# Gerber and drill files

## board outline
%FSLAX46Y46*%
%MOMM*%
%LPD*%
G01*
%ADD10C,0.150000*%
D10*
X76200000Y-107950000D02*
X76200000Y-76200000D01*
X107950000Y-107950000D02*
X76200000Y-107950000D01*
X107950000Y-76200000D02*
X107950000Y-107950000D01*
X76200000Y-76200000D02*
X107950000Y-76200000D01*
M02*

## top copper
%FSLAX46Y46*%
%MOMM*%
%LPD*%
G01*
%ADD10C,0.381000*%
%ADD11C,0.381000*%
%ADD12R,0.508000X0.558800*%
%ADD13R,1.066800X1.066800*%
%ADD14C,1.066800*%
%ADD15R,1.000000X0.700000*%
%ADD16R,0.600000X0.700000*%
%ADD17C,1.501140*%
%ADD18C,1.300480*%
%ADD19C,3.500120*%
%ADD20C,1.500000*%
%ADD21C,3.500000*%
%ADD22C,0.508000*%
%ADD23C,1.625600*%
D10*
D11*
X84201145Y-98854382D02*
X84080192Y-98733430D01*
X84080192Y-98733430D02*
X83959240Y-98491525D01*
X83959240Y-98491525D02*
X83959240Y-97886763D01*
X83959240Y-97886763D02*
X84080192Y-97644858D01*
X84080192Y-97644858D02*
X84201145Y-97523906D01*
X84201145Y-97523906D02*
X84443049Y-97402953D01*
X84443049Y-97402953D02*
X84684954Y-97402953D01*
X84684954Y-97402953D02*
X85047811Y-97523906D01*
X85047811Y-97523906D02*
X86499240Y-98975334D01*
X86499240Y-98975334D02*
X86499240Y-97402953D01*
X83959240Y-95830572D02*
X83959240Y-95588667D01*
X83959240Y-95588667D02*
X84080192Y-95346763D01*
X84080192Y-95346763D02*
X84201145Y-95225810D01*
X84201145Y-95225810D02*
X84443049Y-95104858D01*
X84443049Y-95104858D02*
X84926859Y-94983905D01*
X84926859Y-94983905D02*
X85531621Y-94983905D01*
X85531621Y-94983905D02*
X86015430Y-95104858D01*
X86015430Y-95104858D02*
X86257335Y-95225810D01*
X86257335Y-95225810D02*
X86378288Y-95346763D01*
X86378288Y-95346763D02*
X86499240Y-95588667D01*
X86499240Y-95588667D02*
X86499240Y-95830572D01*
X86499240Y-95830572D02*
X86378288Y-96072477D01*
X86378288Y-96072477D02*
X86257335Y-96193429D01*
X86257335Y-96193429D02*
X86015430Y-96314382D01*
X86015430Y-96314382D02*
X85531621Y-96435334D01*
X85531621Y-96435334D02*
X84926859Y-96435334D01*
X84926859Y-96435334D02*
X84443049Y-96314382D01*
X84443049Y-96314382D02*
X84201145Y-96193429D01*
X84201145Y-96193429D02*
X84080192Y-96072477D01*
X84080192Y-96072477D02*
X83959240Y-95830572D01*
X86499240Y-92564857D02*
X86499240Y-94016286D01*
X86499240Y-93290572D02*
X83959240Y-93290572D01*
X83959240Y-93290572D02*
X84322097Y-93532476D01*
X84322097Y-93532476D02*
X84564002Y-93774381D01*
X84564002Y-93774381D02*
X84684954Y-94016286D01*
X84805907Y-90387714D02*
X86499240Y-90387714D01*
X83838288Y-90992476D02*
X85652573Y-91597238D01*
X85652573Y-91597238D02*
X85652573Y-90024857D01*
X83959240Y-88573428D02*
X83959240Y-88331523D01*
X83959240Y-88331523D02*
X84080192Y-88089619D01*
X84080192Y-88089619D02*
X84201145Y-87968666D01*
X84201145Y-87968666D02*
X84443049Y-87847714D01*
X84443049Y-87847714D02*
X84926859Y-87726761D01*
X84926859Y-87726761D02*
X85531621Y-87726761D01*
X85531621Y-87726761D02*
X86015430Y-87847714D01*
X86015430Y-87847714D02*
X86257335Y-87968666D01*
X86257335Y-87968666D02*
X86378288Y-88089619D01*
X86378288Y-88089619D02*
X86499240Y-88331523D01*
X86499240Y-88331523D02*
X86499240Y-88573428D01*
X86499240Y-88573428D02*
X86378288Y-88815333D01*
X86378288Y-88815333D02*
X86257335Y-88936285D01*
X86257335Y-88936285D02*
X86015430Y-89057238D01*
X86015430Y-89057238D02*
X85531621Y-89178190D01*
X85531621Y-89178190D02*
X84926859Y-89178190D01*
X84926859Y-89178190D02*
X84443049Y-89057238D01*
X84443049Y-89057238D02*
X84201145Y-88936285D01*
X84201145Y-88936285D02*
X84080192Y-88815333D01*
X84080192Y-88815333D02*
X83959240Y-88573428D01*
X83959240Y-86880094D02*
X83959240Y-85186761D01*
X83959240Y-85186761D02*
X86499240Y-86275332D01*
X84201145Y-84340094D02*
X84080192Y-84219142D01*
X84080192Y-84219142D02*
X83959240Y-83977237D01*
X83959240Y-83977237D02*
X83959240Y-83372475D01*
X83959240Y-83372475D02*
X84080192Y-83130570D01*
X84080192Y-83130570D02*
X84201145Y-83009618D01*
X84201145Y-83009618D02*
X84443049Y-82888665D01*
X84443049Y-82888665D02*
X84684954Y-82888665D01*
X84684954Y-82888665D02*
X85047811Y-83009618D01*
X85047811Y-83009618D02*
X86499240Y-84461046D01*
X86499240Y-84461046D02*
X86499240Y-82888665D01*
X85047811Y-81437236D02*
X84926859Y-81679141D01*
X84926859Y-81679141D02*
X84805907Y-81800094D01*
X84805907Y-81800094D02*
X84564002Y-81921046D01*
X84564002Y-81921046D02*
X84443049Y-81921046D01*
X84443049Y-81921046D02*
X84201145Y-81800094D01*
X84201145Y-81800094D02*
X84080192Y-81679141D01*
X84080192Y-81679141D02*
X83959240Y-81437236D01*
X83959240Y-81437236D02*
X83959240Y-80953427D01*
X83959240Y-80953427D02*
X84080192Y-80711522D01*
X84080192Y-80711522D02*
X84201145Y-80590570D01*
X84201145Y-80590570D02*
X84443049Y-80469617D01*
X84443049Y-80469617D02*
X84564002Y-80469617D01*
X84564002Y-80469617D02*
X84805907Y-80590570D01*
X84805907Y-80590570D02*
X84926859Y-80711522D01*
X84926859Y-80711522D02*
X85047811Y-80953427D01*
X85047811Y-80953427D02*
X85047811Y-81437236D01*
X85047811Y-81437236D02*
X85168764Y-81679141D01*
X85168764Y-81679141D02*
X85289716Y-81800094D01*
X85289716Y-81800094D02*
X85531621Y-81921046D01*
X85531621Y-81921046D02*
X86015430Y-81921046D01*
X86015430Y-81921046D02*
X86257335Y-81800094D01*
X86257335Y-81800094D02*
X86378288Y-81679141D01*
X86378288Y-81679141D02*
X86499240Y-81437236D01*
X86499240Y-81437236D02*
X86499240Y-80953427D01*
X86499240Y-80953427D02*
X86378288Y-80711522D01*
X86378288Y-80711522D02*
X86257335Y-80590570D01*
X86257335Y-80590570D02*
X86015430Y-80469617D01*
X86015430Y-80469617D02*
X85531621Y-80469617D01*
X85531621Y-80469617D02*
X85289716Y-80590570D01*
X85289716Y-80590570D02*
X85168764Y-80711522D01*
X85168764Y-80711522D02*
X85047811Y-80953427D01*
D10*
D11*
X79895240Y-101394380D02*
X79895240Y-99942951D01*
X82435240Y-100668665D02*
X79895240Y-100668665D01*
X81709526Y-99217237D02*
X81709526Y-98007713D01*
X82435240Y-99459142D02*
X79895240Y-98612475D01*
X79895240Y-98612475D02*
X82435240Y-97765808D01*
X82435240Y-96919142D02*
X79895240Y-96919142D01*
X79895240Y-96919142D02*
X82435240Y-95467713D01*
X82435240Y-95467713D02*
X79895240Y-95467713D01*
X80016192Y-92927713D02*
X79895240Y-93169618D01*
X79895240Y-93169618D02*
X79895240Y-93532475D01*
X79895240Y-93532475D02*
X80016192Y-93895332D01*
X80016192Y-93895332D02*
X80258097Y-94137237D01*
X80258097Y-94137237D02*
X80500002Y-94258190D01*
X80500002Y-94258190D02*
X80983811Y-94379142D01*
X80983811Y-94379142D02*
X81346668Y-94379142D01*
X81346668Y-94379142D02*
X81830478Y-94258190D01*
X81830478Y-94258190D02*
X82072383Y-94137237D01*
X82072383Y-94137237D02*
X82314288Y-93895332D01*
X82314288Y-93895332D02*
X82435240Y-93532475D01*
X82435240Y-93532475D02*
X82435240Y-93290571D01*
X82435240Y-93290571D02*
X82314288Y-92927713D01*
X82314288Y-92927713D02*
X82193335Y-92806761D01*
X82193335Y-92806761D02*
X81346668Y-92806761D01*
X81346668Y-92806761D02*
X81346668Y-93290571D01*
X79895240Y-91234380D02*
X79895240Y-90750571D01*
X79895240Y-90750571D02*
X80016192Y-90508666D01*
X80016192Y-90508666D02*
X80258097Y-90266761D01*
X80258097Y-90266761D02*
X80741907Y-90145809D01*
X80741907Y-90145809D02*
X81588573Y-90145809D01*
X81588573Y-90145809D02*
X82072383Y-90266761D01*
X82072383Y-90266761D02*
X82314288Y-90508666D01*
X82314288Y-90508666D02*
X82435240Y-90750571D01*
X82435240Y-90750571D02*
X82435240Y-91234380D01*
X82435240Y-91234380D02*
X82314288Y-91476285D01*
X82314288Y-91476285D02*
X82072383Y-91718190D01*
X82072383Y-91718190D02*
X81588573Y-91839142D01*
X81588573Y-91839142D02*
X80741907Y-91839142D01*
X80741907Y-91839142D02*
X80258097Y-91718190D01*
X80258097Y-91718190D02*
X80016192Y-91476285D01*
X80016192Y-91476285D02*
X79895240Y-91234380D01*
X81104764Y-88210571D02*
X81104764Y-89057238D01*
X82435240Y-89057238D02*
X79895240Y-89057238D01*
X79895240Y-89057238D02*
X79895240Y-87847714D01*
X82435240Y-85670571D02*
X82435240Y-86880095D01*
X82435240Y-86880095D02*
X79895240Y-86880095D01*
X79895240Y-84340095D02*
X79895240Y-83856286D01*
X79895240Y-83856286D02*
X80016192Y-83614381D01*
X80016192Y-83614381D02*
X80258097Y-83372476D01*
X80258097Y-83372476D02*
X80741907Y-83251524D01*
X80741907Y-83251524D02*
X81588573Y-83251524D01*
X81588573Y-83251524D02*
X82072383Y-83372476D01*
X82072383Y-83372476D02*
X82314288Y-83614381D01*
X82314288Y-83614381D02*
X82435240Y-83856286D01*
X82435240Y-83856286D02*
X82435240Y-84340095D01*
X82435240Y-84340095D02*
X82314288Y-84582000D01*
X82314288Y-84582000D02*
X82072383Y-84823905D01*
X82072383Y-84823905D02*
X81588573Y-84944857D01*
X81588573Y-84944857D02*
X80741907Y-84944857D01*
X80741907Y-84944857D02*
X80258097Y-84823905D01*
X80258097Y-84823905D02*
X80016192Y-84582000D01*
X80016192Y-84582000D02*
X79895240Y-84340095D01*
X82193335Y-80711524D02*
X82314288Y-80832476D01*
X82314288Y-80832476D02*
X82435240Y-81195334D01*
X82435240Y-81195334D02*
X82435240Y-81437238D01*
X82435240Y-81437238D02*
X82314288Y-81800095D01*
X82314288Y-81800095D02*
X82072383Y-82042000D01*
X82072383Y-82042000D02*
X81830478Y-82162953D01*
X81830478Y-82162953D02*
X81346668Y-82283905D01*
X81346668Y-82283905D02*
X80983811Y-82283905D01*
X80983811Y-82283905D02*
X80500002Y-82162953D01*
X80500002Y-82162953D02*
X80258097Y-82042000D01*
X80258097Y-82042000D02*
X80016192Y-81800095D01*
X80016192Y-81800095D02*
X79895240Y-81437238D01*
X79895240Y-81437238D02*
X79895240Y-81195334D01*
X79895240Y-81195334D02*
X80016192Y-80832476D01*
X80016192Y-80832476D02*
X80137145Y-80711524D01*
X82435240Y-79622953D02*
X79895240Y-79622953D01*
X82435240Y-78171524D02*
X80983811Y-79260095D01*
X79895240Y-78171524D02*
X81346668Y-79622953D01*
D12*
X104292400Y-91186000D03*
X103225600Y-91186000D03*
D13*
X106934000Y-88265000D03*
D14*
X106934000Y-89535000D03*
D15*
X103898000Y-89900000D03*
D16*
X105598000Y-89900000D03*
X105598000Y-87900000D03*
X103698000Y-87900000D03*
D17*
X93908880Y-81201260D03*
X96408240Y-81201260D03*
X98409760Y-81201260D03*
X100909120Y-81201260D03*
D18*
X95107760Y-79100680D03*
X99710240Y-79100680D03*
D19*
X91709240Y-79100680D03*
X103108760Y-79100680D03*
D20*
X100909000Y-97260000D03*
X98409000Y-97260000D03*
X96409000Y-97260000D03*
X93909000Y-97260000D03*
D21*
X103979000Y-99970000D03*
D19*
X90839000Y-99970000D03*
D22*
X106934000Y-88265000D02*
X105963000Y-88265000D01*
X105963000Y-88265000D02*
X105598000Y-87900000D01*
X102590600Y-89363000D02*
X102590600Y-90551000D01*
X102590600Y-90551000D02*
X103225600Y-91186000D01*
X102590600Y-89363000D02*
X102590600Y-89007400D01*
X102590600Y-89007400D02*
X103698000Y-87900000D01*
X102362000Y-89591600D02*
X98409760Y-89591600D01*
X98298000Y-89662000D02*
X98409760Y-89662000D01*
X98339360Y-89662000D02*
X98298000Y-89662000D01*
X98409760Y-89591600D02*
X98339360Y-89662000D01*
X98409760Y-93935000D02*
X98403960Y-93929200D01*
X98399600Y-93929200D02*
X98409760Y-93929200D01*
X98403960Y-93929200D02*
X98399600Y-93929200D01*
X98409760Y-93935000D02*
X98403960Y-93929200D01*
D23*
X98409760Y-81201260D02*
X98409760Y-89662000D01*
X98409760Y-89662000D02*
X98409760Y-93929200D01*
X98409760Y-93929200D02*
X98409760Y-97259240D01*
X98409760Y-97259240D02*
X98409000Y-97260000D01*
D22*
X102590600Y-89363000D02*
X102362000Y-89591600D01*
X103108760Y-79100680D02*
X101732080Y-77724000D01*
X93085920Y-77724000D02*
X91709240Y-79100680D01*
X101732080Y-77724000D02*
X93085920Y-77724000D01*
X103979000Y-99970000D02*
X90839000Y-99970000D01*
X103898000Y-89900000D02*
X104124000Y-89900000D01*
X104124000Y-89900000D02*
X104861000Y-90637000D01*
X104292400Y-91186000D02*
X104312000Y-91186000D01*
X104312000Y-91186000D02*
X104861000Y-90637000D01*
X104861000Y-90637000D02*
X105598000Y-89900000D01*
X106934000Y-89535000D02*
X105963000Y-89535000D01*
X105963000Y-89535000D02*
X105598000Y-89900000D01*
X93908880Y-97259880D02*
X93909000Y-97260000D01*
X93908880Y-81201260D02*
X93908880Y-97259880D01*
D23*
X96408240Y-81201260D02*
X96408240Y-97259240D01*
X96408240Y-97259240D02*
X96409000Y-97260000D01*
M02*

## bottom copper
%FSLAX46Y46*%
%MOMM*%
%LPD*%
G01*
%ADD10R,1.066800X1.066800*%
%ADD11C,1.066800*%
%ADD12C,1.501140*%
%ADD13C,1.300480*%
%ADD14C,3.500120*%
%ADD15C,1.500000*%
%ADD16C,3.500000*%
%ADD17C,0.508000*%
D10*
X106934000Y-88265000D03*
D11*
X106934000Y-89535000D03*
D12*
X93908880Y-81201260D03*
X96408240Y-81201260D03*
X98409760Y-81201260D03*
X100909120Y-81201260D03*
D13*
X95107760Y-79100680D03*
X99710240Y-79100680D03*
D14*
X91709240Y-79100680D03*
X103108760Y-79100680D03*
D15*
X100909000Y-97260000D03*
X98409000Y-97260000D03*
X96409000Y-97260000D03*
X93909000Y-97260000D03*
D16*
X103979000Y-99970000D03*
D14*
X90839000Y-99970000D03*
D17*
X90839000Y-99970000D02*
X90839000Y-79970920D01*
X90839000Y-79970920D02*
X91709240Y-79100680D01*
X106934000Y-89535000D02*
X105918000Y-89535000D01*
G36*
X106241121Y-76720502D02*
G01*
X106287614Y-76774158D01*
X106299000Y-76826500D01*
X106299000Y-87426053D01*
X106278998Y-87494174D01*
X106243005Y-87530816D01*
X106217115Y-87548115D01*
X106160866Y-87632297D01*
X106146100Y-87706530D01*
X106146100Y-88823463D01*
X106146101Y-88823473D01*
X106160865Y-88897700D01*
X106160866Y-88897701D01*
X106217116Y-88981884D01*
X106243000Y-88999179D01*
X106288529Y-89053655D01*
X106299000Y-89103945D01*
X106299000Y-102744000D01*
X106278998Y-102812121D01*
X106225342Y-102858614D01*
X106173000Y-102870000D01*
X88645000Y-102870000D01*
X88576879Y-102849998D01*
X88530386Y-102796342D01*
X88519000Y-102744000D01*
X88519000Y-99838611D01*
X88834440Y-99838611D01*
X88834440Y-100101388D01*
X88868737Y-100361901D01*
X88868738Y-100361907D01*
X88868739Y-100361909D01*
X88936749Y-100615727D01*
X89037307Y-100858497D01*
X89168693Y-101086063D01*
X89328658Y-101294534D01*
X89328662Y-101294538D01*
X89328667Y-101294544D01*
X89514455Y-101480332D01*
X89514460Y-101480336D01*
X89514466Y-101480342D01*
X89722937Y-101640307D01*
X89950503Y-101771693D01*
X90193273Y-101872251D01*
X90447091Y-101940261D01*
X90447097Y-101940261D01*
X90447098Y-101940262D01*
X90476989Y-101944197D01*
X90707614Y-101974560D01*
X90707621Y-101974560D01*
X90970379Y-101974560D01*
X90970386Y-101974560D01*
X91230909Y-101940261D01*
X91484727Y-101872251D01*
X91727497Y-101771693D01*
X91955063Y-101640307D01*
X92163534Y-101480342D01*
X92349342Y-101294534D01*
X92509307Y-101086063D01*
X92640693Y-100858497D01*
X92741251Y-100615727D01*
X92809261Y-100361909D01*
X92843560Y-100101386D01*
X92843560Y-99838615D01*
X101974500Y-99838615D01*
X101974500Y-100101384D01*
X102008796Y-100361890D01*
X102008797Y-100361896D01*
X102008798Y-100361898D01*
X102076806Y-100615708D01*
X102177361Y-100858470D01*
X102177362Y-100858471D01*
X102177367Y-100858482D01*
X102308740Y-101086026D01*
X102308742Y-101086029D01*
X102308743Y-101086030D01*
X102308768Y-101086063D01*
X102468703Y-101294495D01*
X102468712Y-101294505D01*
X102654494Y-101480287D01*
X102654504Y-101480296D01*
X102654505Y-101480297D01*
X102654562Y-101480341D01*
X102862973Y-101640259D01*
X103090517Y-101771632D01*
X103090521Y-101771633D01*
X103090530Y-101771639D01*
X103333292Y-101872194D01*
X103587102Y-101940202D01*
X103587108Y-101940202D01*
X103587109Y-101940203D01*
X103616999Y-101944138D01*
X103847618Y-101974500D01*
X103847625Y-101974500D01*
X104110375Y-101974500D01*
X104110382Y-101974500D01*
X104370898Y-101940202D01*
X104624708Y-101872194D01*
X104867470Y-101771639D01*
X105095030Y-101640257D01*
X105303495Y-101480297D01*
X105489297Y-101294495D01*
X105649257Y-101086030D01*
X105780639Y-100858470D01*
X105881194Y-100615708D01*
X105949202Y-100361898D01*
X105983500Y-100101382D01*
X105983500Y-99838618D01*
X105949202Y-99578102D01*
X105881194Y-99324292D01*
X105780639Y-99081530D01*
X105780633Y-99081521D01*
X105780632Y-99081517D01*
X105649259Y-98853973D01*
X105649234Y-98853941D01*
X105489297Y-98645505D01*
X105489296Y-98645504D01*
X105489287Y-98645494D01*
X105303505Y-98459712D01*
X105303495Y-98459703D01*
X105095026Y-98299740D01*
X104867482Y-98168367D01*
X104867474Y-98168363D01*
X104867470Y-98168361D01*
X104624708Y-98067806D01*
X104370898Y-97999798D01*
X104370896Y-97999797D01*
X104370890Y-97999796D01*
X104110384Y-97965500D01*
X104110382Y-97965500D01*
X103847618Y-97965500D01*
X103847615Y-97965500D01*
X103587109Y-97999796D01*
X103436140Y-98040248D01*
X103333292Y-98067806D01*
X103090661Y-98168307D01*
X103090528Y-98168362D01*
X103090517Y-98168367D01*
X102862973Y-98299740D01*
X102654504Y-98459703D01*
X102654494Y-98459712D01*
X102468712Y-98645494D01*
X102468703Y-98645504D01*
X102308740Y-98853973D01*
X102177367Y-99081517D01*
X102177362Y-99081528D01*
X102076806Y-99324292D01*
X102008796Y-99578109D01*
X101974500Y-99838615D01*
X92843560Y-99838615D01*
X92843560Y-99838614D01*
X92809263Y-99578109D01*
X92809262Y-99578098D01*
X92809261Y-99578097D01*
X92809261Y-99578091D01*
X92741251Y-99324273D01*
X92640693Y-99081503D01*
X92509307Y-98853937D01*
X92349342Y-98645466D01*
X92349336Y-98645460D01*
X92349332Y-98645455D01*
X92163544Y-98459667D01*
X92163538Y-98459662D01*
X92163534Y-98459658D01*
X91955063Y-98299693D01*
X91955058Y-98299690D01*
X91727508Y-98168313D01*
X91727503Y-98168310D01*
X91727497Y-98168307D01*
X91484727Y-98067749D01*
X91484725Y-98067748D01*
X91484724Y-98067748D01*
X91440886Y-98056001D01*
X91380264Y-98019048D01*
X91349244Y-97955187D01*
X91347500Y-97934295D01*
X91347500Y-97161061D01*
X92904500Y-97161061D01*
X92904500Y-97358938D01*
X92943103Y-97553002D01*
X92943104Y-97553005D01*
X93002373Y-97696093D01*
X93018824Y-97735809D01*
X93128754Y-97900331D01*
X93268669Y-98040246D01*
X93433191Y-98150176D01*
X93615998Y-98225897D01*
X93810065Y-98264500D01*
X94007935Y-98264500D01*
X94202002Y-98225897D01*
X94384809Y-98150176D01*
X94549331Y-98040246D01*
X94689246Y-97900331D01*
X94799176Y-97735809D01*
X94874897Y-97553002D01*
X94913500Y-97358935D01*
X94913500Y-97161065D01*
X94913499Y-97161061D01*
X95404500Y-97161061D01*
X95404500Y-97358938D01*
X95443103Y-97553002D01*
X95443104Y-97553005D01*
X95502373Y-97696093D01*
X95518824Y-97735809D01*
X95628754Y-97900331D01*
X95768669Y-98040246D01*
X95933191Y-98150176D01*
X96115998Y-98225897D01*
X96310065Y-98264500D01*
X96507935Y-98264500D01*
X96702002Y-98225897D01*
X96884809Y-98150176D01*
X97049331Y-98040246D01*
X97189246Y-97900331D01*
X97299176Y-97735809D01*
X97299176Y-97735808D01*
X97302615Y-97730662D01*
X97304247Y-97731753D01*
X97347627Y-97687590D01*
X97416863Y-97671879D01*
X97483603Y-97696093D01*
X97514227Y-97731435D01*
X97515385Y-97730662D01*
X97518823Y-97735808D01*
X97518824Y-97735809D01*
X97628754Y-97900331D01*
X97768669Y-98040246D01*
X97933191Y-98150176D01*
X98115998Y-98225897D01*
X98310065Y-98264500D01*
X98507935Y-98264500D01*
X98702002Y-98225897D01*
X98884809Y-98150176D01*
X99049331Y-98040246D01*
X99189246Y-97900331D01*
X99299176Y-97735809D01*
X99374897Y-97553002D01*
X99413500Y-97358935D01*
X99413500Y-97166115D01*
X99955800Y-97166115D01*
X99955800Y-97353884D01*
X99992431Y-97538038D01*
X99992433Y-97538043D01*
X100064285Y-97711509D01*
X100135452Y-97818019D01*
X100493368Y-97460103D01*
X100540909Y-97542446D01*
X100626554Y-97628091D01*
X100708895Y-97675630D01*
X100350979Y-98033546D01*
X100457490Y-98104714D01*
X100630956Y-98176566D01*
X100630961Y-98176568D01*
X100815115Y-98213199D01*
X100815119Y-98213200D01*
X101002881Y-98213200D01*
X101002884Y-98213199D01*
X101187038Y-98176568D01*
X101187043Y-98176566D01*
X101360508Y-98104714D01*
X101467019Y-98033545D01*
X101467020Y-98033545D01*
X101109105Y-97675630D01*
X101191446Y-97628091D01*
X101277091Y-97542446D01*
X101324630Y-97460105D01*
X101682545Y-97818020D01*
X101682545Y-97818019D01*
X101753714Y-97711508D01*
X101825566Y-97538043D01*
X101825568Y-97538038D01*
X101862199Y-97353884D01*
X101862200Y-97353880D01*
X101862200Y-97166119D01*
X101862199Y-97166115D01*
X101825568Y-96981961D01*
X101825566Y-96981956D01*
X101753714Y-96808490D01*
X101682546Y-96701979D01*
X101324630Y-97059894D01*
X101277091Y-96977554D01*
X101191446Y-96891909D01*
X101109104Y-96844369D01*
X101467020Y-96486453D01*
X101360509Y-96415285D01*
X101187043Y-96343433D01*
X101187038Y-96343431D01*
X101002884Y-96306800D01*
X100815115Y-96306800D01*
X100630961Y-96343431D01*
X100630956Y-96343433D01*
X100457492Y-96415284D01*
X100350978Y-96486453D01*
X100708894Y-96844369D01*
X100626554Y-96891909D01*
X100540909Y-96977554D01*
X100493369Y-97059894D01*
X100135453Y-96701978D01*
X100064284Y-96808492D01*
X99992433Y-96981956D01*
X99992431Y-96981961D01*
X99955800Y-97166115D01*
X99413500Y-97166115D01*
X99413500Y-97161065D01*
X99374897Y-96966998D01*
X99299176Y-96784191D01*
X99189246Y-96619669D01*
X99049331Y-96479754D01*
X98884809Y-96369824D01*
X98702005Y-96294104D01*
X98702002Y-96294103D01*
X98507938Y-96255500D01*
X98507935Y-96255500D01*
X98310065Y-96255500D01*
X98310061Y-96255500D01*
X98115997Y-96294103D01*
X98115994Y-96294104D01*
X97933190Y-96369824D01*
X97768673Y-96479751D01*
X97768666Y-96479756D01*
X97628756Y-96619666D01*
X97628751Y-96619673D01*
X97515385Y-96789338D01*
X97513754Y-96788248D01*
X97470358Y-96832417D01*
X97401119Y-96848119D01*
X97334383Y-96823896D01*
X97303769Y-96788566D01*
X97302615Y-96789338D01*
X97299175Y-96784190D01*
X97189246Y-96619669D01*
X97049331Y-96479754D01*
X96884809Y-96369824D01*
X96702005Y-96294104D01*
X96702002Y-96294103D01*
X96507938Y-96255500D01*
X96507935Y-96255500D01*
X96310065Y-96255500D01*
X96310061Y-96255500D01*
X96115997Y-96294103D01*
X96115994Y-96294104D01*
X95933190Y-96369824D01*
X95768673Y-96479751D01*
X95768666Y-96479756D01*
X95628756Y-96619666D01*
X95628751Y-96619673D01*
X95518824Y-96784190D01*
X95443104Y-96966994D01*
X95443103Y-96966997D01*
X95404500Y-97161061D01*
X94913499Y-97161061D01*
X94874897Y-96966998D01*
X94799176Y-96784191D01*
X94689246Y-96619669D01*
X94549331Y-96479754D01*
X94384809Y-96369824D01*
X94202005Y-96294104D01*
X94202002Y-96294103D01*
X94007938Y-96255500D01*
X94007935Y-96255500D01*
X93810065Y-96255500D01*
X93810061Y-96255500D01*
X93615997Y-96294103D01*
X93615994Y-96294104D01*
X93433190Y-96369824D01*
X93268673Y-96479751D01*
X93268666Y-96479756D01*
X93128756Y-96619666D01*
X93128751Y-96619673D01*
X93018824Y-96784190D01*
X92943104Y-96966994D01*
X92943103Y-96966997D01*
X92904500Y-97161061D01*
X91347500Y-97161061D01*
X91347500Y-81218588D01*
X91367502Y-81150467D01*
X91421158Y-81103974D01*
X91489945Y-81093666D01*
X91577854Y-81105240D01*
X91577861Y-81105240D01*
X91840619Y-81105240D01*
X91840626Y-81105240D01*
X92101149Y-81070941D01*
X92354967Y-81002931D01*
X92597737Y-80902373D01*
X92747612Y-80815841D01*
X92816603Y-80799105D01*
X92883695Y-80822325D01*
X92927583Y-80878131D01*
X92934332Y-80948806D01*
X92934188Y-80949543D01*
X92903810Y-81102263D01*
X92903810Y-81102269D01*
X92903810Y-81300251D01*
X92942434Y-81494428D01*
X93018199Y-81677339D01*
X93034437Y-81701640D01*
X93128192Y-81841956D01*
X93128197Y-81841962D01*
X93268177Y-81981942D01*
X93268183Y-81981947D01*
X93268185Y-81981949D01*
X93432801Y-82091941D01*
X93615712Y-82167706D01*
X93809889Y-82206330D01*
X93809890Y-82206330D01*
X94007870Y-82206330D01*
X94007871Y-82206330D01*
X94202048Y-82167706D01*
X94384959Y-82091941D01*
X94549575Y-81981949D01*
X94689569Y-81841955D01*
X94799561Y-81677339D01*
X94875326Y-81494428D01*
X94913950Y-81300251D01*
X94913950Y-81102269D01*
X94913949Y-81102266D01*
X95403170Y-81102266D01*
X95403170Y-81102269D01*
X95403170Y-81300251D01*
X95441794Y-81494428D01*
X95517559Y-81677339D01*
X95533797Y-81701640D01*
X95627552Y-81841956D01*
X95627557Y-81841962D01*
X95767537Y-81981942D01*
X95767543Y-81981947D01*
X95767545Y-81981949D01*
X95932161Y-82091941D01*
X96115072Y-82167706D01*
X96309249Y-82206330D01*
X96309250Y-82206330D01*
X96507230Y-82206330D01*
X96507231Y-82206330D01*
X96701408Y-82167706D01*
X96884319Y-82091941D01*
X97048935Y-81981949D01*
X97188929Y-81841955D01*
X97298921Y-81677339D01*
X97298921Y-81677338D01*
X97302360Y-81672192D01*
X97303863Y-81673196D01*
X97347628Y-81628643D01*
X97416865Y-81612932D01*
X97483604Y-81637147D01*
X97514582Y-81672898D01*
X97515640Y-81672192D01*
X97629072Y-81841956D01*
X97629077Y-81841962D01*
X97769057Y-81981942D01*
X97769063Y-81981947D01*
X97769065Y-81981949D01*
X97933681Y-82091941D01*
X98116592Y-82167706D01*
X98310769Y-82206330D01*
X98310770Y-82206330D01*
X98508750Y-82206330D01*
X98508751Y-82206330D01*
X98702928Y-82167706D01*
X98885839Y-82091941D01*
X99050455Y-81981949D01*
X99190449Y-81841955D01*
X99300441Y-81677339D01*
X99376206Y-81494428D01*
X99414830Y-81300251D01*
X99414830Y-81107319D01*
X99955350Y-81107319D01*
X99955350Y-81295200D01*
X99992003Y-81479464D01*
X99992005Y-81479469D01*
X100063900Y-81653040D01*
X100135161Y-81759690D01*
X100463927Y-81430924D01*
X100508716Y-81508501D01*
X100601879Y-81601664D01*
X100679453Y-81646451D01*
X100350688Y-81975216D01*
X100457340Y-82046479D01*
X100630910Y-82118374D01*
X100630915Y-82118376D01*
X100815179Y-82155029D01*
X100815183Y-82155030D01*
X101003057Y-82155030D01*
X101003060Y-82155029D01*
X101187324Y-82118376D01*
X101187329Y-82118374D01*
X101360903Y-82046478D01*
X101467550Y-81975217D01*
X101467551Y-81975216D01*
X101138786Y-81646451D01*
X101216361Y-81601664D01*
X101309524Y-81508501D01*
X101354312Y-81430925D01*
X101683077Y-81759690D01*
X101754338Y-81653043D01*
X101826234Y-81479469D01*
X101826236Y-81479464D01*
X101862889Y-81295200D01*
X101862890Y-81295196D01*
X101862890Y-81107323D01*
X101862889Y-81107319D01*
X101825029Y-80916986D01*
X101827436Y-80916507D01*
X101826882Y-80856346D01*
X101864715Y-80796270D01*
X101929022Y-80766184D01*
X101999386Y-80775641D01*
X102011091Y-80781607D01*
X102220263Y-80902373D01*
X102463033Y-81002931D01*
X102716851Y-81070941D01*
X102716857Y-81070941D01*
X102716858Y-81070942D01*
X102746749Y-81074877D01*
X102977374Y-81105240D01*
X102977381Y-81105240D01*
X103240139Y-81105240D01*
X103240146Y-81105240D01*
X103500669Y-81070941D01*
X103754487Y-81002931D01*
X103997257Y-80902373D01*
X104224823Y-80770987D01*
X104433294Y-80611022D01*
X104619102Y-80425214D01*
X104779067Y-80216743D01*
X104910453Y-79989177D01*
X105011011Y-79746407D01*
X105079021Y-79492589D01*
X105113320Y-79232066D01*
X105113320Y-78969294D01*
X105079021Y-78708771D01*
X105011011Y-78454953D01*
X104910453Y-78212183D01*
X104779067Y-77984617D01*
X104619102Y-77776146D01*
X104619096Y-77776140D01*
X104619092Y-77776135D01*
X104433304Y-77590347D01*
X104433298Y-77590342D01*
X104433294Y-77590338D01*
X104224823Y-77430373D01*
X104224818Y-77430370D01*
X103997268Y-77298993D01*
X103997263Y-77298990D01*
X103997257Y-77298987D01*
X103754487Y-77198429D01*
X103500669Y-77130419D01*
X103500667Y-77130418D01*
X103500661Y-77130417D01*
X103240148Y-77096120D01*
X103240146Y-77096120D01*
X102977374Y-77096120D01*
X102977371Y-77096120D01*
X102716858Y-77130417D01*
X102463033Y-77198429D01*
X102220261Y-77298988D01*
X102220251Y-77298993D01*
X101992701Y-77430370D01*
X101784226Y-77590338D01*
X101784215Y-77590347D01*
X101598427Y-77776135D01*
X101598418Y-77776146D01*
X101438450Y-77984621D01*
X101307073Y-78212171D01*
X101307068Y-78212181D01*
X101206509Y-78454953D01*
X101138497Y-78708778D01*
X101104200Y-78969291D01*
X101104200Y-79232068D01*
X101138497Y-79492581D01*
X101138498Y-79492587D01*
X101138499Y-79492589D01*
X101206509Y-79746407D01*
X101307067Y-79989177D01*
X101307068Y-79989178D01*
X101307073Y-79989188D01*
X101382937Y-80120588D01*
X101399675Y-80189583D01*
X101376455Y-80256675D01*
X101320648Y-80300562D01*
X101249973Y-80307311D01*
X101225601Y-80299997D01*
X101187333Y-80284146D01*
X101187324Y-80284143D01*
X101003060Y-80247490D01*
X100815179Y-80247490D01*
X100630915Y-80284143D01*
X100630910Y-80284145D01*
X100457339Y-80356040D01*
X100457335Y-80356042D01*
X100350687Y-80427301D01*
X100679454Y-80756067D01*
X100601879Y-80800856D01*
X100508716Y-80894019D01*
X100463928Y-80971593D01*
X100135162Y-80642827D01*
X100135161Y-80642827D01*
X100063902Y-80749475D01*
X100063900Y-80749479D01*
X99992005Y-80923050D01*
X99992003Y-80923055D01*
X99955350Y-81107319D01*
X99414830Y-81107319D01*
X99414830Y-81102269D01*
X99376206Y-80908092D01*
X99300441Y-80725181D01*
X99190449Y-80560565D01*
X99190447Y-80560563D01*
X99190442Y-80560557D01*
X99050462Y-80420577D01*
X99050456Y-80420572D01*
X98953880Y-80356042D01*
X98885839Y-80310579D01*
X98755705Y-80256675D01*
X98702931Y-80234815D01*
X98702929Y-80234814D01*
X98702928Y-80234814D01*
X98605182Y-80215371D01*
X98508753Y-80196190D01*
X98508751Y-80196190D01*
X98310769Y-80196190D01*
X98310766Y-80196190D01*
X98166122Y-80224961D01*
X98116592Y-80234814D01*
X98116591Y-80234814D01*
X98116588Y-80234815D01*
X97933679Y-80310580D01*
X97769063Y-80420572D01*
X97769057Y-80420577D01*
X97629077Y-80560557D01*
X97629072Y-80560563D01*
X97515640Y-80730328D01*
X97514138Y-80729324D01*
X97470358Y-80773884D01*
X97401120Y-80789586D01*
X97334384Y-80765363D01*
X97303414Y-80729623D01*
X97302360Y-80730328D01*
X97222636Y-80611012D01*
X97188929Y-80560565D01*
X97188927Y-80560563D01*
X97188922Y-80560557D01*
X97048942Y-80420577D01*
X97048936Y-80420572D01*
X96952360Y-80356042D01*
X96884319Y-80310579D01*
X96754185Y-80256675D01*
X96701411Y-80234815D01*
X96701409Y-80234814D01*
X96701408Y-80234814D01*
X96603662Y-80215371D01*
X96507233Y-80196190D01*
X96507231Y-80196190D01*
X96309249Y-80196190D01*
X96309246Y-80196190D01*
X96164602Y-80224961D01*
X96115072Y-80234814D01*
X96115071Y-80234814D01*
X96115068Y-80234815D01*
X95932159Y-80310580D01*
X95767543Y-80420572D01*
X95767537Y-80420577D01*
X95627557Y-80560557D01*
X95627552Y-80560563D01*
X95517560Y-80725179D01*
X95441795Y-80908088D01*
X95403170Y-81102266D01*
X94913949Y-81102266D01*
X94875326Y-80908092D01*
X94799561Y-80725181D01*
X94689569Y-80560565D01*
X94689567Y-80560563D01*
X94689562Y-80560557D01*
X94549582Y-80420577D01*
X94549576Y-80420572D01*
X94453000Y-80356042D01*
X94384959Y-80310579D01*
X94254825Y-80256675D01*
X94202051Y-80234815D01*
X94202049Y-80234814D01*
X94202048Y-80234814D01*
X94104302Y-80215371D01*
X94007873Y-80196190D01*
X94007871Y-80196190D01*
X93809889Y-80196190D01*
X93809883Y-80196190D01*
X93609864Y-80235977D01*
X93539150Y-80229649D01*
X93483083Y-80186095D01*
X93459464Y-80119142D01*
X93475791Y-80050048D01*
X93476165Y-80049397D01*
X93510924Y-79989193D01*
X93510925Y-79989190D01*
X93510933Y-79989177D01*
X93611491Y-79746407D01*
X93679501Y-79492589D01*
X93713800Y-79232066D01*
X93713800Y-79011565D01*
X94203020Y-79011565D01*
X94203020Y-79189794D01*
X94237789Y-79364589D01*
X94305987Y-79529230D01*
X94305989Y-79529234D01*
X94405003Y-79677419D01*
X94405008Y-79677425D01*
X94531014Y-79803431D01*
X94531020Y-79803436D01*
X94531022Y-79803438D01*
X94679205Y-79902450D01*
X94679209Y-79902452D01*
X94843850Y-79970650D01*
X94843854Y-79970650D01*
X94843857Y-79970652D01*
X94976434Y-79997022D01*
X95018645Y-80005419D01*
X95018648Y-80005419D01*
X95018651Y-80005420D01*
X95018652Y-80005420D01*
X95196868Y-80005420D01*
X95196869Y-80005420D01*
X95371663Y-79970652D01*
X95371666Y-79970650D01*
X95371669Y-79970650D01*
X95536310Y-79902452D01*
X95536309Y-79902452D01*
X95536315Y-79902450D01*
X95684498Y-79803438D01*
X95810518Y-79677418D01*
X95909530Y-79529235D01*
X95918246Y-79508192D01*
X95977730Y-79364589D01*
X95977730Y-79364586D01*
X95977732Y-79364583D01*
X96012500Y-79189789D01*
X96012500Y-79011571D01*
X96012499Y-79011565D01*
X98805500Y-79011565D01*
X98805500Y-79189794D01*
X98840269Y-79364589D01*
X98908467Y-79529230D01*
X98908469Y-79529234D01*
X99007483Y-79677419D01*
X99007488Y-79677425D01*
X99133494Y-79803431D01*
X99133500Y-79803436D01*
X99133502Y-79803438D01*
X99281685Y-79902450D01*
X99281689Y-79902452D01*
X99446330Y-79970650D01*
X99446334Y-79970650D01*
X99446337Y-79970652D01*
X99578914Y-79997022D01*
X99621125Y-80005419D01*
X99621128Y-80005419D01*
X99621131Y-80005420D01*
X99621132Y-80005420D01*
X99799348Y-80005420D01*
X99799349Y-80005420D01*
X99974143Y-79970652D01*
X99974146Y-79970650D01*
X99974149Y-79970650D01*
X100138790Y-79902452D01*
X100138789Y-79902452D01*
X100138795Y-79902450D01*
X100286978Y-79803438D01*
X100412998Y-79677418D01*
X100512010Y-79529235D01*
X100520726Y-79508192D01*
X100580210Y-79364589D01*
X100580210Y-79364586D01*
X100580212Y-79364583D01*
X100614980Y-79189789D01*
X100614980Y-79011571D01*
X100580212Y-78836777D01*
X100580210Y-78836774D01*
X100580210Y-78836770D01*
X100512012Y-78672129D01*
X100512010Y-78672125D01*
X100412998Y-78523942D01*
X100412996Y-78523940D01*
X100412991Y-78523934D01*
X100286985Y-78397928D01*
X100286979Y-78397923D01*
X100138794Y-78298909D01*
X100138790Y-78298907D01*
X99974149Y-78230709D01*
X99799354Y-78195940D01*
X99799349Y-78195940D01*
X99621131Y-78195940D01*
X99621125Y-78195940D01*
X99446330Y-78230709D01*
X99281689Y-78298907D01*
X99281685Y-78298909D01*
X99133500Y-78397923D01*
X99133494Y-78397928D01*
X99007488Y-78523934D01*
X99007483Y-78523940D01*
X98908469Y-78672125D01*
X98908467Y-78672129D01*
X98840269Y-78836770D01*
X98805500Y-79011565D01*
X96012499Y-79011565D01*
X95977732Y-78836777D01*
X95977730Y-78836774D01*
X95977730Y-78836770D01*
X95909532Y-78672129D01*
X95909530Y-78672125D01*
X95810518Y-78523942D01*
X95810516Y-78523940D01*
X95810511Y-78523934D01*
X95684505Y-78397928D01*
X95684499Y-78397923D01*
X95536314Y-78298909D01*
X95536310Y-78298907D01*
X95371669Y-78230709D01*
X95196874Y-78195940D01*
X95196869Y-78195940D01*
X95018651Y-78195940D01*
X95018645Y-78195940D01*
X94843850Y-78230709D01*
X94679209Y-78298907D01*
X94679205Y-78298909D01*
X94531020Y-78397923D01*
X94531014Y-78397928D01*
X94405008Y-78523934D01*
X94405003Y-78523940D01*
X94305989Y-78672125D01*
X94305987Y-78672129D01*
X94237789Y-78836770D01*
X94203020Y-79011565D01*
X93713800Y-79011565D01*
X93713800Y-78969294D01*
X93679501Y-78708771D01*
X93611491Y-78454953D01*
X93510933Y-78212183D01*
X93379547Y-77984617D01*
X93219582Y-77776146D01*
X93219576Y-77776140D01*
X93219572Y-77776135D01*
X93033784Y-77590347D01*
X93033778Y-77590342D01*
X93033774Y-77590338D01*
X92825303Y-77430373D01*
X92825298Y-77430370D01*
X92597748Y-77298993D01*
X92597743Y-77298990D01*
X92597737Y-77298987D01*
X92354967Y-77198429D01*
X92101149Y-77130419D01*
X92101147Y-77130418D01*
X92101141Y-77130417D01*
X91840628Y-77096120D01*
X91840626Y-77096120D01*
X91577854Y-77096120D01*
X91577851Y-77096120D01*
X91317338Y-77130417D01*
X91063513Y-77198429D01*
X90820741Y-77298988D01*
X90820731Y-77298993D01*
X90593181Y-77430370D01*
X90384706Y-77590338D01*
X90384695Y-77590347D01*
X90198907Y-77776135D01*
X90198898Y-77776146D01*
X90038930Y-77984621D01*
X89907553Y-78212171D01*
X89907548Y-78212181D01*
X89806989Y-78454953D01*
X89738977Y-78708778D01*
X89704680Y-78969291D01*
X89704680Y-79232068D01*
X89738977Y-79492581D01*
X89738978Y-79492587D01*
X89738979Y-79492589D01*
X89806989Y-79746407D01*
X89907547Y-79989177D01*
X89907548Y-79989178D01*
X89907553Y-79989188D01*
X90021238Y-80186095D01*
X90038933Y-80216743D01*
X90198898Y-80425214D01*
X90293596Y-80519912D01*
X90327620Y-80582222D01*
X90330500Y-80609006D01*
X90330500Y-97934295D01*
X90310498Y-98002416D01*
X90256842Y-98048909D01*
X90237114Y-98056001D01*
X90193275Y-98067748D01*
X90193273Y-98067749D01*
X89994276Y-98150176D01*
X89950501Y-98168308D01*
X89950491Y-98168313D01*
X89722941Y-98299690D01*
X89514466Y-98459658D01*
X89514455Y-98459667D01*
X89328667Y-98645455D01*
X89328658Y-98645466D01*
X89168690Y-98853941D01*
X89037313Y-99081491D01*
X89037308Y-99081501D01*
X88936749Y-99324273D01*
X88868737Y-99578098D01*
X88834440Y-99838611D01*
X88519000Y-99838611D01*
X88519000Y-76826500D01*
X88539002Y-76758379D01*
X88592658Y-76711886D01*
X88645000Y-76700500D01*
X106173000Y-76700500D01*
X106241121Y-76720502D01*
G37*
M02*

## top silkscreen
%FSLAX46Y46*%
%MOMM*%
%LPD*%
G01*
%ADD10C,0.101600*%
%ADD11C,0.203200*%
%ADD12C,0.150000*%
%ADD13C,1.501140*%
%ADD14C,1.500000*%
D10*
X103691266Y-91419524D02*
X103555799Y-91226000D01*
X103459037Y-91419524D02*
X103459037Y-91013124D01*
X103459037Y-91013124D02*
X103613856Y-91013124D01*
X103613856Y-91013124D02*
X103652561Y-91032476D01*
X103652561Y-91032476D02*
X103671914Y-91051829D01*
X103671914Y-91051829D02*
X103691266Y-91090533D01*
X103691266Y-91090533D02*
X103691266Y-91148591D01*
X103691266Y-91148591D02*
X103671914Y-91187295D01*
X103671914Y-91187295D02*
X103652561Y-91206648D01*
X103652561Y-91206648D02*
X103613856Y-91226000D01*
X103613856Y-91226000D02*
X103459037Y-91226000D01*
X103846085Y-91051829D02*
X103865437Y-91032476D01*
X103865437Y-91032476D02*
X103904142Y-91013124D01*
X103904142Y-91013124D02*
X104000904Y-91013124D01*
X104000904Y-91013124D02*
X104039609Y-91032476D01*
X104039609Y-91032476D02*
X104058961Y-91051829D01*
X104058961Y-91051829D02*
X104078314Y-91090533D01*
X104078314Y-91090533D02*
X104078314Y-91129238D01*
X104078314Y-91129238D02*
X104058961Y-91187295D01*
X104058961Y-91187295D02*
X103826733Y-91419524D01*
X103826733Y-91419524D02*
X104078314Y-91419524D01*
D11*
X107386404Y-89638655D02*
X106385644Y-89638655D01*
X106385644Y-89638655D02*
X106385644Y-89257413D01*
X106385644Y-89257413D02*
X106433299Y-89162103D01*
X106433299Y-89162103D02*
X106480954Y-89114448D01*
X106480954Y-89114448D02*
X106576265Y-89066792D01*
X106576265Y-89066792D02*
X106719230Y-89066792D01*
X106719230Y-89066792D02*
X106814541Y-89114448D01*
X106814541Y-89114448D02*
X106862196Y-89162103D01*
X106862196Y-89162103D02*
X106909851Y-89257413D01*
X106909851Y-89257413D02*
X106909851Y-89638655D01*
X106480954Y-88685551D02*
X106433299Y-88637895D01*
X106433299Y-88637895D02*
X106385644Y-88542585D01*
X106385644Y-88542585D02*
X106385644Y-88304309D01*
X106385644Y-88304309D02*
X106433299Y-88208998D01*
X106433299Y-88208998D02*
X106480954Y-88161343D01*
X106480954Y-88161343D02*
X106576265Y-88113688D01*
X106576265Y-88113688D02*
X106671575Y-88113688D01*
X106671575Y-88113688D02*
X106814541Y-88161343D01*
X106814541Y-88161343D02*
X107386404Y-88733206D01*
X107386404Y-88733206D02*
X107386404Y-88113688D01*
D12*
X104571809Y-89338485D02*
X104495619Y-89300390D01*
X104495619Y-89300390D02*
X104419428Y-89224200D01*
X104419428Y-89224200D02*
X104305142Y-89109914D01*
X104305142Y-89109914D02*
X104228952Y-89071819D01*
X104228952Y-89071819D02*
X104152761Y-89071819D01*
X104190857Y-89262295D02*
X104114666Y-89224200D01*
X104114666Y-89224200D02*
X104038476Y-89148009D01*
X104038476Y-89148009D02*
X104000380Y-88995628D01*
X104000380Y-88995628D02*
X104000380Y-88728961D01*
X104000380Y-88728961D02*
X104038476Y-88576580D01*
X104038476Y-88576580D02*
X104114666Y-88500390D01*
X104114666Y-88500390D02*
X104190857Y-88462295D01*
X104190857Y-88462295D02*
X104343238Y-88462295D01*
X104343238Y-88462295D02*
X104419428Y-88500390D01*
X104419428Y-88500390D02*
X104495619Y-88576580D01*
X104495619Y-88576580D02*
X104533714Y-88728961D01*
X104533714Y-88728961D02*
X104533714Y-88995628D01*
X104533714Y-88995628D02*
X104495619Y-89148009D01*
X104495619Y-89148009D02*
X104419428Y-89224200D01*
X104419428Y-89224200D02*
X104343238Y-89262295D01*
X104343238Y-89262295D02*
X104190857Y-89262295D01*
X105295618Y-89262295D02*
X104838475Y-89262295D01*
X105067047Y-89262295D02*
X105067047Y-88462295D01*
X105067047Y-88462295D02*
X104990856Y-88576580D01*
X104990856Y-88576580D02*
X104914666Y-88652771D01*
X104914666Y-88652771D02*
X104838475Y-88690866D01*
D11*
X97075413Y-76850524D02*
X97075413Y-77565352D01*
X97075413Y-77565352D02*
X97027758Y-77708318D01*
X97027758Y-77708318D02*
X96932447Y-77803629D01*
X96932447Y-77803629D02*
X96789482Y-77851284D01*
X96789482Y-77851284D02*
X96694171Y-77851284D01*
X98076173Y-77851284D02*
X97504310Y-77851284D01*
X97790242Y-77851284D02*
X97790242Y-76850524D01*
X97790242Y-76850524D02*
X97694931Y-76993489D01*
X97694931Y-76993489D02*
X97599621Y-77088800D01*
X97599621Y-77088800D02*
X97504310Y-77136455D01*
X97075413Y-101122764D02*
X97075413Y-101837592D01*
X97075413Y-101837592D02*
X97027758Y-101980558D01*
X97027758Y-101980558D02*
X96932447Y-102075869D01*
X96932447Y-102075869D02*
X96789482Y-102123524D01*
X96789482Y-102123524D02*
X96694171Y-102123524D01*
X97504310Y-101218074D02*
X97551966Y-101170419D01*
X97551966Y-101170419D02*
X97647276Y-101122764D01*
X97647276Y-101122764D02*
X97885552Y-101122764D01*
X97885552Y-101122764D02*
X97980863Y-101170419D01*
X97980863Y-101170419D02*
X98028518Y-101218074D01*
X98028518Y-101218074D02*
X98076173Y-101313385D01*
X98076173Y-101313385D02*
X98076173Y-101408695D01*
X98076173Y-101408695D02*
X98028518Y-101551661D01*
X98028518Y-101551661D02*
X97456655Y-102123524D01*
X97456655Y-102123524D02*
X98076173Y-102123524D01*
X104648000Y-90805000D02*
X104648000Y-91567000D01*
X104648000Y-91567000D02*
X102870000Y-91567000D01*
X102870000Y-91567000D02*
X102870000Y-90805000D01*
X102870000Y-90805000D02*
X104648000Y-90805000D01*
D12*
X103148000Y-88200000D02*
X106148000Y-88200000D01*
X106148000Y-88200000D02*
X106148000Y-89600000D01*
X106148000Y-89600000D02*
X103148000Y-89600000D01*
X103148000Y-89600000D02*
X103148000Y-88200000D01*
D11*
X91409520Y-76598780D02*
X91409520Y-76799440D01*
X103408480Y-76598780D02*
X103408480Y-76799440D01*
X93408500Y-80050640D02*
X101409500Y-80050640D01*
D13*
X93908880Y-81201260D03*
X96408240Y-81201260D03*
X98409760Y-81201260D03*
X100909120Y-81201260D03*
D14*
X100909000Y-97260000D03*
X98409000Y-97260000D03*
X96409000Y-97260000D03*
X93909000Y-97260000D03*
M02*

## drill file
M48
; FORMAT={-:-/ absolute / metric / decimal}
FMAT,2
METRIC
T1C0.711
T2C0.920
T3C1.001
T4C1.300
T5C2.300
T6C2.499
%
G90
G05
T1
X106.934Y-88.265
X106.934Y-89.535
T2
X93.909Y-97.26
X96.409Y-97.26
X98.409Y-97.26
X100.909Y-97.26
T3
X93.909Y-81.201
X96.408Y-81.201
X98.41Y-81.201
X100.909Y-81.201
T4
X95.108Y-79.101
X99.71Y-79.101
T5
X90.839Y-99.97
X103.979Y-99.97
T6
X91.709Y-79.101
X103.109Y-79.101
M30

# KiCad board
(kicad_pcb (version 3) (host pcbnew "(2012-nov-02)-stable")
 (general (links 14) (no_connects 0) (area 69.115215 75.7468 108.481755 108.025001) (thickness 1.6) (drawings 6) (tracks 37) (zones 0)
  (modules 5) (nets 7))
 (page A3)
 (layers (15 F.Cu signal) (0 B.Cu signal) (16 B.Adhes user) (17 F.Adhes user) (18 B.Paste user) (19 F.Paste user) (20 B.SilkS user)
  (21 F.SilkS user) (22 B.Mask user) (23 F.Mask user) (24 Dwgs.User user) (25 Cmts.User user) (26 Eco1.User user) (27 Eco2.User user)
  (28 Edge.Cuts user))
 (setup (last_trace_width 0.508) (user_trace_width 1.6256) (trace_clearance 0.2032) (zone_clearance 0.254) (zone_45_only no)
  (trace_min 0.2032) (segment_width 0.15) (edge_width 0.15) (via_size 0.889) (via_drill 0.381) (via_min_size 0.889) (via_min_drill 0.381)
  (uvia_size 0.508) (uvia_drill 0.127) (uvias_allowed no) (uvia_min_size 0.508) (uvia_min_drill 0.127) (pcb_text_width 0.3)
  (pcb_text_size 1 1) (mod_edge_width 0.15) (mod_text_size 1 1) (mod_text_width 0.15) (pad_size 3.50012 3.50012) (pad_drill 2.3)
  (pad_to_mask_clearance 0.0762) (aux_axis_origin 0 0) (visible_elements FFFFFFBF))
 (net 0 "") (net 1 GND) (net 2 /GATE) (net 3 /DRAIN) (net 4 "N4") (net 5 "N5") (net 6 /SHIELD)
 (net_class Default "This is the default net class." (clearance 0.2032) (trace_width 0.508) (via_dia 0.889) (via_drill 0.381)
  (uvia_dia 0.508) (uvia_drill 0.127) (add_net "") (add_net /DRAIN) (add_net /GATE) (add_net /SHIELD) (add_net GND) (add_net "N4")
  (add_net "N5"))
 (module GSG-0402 (layer F.Cu) (at 103.759 91.186) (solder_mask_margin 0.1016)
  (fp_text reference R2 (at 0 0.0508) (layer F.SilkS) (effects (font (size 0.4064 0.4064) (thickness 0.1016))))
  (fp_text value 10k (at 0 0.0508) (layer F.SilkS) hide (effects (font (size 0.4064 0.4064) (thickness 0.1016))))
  (fp_line (start 0.889 -0.381) (end 0.889 0.381) (layer F.SilkS) (width 0.2032))
  (fp_line (start 0.889 0.381) (end -0.889 0.381) (layer F.SilkS) (width 0.2032))
  (fp_line (start -0.889 0.381) (end -0.889 -0.381) (layer F.SilkS) (width 0.2032))
  (fp_line (start -0.889 -0.381) (end 0.889 -0.381) (layer F.SilkS) (width 0.2032))
  (pad 2 smd rect (at 0.5334 0) (size 0.508 0.5588) (layers F.Cu F.Paste F.Mask) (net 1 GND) (solder_mask_margin 0.1016))
  (pad 1 smd rect (at -0.5334 0) (size 0.508 0.5588) (layers F.Cu F.Paste F.Mask) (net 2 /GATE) (die_length -2147.483648)
   (solder_mask_margin 0.1016)))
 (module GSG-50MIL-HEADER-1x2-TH (layer F.Cu) (at 106.934 88.9 270)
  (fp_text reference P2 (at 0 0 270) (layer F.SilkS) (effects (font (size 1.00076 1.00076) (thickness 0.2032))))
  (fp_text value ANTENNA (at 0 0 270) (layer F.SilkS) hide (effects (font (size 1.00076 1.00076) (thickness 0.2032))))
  (pad 1 thru_hole rect (at -0.635 0 270) (size 1.0668 1.0668) (drill 0.7112) (layers *.Cu *.Mask) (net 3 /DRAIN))
  (pad 2 thru_hole circle (at 0.635 0 270) (size 1.0668 1.0668) (drill 0.7112) (layers *.Cu *.Mask) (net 1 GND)))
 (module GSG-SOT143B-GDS (layer F.Cu) (at 104.648 88.9)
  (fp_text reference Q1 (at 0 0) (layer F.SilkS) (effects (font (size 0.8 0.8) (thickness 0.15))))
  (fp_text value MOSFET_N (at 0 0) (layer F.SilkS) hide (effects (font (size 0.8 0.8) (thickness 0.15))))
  (fp_line (start -1.5 -0.7) (end 1.5 -0.7) (layer F.SilkS) (width 0.15))
  (fp_line (start 1.5 -0.7) (end 1.5 0.7) (layer F.SilkS) (width 0.15))
  (fp_line (start 1.5 0.7) (end -1.5 0.7) (layer F.SilkS) (width 0.15))
  (fp_line (start -1.5 0.7) (end -1.5 -0.7) (layer F.SilkS) (width 0.15))
  (pad B smd rect (at -0.75 1) (size 1 0.7) (layers F.Cu F.Paste F.Mask) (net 1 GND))
  (pad S smd rect (at 0.95 1) (size 0.6 0.7) (layers F.Cu F.Paste F.Mask) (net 1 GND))
  (pad D smd rect (at 0.95 -1) (size 0.6 0.7) (layers F.Cu F.Paste F.Mask) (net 3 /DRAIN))
  (pad G smd rect (at -0.95 -1) (size 0.6 0.7) (layers F.Cu F.Paste F.Mask) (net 2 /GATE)))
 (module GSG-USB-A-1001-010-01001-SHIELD (layer F.Cu) (at 97.409 76.2 180)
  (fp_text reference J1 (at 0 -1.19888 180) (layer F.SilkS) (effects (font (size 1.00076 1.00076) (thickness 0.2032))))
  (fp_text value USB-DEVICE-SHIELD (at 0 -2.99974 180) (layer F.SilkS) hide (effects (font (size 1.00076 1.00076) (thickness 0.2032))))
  (fp_line (start 5.99948 -0.39878) (end 5.99948 -0.59944) (layer F.SilkS) (width 0.2032))
  (fp_line (start -5.99948 -0.39878) (end -5.99948 -0.59944) (layer F.SilkS) (width 0.2032))
  (fp_line (start 4.0005 -3.85064) (end -4.0005 -3.85064) (layer F.SilkS) (width 0.2032))
  (pad 1 thru_hole circle (at 3.50012 -5.00126 180) (size 1.50114 1.50114) (drill 1.00076) (layers *.Cu *.Mask F.SilkS) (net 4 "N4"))
  (pad 2 thru_hole circle (at 1.00076 -5.00126 180) (size 1.50114 1.50114) (drill 1.00076) (layers *.Cu *.Mask F.SilkS) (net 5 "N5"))
  (pad 3 thru_hole circle (at -1.00076 -5.00126 180) (size 1.50114 1.50114) (drill 1.00076) (layers *.Cu *.Mask F.SilkS) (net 2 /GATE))
  (pad 4 thru_hole circle (at -3.50012 -5.00126 180) (size 1.50114 1.50114) (drill 1.00076) (layers *.Cu *.Mask F.SilkS) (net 1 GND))
  (pad "" thru_hole circle (at 2.30124 -2.90068 180) (size 1.30048 1.30048) (drill 1.30048) (layers *.Cu *.Mask) (clearance -0.09906))
  (pad "" thru_hole circle (at -2.30124 -2.90068 180) (size 1.30048 1.30048) (drill 1.30048) (layers *.Cu *.Mask) (clearance -0.09906))
  (pad 5 thru_hole circle (at 5.69976 -2.90068 180) (size 3.50012 3.50012) (drill 2.49936) (layers *.Cu *.Mask) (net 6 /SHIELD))
  (pad 5 thru_hole circle (at -5.69976 -2.90068 180) (size 3.50012 3.50012) (drill 2.49936) (layers *.Cu *.Mask) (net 6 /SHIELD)))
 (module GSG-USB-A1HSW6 (layer F.Cu) (at 97.409 102.87)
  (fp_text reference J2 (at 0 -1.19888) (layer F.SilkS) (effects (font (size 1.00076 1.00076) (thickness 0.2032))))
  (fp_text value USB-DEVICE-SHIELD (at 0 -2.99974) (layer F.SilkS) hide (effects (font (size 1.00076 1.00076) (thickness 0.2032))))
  (pad 4 thru_hole circle (at 3.5 -5.61) (size 1.5 1.5) (drill 0.92) (layers *.Cu *.Mask F.SilkS) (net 1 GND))
  (pad 3 thru_hole circle (at 1 -5.61) (size 1.5 1.5) (drill 0.92) (layers *.Cu *.Mask F.SilkS) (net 2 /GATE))
  (pad 2 thru_hole circle (at -1 -5.61) (size 1.5 1.5) (drill 0.92) (layers *.Cu *.Mask F.SilkS) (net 5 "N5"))
  (pad 1 thru_hole circle (at -3.5 -5.61) (size 1.5 1.5) (drill 0.92) (layers *.Cu *.Mask F.SilkS) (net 4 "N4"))
  (pad 5 thru_hole circle (at 6.57 -2.9) (size 3.5 3.5) (drill 2.3) (layers *.Cu *.Mask) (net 6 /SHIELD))
  (pad 5 thru_hole circle (at -6.57 -2.9) (size 3.50012 3.50012) (drill 2.3) (layers *.Cu *.Mask) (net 6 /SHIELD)))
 (gr_line (start 76.2 107.95) (end 76.2 76.2) (angle 90) (layer Edge.Cuts) (width 0.15))
 (gr_line (start 107.95 107.95) (end 76.2 107.95) (angle 90) (layer Edge.Cuts) (width 0.15))
 (gr_line (start 107.95 76.2) (end 107.95 107.95) (angle 90) (layer Edge.Cuts) (width 0.15))
 (gr_line (start 76.2 76.2) (end 107.95 76.2) (angle 90) (layer Edge.Cuts) (width 0.15))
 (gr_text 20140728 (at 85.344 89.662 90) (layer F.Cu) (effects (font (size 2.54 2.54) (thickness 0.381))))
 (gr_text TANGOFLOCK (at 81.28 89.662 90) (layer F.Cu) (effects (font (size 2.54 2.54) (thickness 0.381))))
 (segment (start 106.934 88.265) (end 105.963 88.265) (width 0.508) (layer F.Cu) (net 3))
 (segment (start 105.963 88.265) (end 105.598 87.9) (width 0.508) (layer F.Cu) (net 3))
 (segment (start 102.5906 89.363) (end 102.5906 90.551) (width 0.508) (layer F.Cu) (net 2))
 (segment (start 102.5906 90.551) (end 103.2256 91.186) (width 0.508) (layer F.Cu) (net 2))
 (segment (start 102.5906 89.363) (end 102.5906 89.0074) (width 0.508) (layer F.Cu) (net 2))
 (segment (start 102.5906 89.0074) (end 103.698 87.9) (width 0.508) (layer F.Cu) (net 2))
 (segment (start 102.362 89.5916) (end 98.40976 89.5916) (width 0.508) (layer F.Cu) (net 2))
 (segment (start 98.298 89.662) (end 98.40976 89.662) (width 0.508) (layer F.Cu) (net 2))
 (segment (start 98.33936 89.662) (end 98.298 89.662) (width 0.508) (layer F.Cu) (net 2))
 (segment (start 98.40976 89.5916) (end 98.33936 89.662) (width 0.508) (layer F.Cu) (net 2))
 (segment (start 98.40976 93.935) (end 98.40396 93.9292) (width 0.508) (layer F.Cu) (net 2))
 (segment (start 98.3996 93.9292) (end 98.40976 93.9292) (width 0.508) (layer F.Cu) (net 2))
 (segment (start 98.40396 93.9292) (end 98.3996 93.9292) (width 0.508) (layer F.Cu) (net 2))
 (segment (start 98.40976 93.935) (end 98.40396 93.9292) (width 0.508) (layer F.Cu) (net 2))
 (segment (start 98.40976 81.20126) (end 98.40976 89.662) (width 1.6256) (layer F.Cu) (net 2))
 (segment (start 98.40976 89.662) (end 98.40976 93.9292) (width 1.6256) (layer F.Cu) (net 2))
 (segment (start 98.40976 93.9292) (end 98.40976 97.25924) (width 1.6256) (layer F.Cu) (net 2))
 (segment (start 98.40976 97.25924) (end 98.409 97.26) (width 1.6256) (layer F.Cu) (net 2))
 (segment (start 102.5906 89.363) (end 102.362 89.5916) (width 0.508) (layer F.Cu) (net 2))
 (segment (start 103.10876 79.10068) (end 101.73208 77.724) (width 0.508) (layer F.Cu) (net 6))
 (segment (start 93.08592 77.724) (end 91.70924 79.10068) (width 0.508) (layer F.Cu) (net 6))
 (segment (start 101.73208 77.724) (end 93.08592 77.724) (width 0.508) (layer F.Cu) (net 6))
 (segment (start 103.979 99.97) (end 90.839 99.97) (width 0.508) (layer F.Cu) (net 6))
 (segment (start 90.839 99.97) (end 90.839 79.97092) (width 0.508) (layer B.Cu) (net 6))
 (segment (start 90.839 79.97092) (end 91.70924 79.10068) (width 0.508) (layer B.Cu) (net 6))
 (segment (start 103.898 89.9) (end 104.124 89.9) (width 0.508) (layer F.Cu) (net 1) (status C00000))
 (segment (start 104.124 89.9) (end 104.861 90.637) (width 0.508) (layer F.Cu) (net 1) (status 400000))
 (segment (start 104.2924 91.186) (end 104.312 91.186) (width 0.508) (layer F.Cu) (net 1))
 (segment (start 104.312 91.186) (end 104.861 90.637) (width 0.508) (layer F.Cu) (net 1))
 (segment (start 104.861 90.637) (end 105.598 89.9) (width 0.508) (layer F.Cu) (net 1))
 (segment (start 106.934 89.535) (end 105.963 89.535) (width 0.508) (layer F.Cu) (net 1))
 (segment (start 105.963 89.535) (end 105.598 89.9) (width 0.508) (layer F.Cu) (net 1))
 (segment (start 106.934 89.535) (end 105.918 89.535) (width 0.508) (layer B.Cu) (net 1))
 (segment (start 93.90888 97.25988) (end 93.909 97.26) (width 0.508) (layer F.Cu) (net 4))
 (segment (start 93.90888 81.20126) (end 93.90888 97.25988) (width 0.508) (layer F.Cu) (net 4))
 (segment (start 96.40824 81.20126) (end 96.40824 97.25924) (width 1.6256) (layer F.Cu) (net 5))
 (segment (start 96.40824 97.25924) (end 96.409 97.26) (width 1.6256) (layer F.Cu) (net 5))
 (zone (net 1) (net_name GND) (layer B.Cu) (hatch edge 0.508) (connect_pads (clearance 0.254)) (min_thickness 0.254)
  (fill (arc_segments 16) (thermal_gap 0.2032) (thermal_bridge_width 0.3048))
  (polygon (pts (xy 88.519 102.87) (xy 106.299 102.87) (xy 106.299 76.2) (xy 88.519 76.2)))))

